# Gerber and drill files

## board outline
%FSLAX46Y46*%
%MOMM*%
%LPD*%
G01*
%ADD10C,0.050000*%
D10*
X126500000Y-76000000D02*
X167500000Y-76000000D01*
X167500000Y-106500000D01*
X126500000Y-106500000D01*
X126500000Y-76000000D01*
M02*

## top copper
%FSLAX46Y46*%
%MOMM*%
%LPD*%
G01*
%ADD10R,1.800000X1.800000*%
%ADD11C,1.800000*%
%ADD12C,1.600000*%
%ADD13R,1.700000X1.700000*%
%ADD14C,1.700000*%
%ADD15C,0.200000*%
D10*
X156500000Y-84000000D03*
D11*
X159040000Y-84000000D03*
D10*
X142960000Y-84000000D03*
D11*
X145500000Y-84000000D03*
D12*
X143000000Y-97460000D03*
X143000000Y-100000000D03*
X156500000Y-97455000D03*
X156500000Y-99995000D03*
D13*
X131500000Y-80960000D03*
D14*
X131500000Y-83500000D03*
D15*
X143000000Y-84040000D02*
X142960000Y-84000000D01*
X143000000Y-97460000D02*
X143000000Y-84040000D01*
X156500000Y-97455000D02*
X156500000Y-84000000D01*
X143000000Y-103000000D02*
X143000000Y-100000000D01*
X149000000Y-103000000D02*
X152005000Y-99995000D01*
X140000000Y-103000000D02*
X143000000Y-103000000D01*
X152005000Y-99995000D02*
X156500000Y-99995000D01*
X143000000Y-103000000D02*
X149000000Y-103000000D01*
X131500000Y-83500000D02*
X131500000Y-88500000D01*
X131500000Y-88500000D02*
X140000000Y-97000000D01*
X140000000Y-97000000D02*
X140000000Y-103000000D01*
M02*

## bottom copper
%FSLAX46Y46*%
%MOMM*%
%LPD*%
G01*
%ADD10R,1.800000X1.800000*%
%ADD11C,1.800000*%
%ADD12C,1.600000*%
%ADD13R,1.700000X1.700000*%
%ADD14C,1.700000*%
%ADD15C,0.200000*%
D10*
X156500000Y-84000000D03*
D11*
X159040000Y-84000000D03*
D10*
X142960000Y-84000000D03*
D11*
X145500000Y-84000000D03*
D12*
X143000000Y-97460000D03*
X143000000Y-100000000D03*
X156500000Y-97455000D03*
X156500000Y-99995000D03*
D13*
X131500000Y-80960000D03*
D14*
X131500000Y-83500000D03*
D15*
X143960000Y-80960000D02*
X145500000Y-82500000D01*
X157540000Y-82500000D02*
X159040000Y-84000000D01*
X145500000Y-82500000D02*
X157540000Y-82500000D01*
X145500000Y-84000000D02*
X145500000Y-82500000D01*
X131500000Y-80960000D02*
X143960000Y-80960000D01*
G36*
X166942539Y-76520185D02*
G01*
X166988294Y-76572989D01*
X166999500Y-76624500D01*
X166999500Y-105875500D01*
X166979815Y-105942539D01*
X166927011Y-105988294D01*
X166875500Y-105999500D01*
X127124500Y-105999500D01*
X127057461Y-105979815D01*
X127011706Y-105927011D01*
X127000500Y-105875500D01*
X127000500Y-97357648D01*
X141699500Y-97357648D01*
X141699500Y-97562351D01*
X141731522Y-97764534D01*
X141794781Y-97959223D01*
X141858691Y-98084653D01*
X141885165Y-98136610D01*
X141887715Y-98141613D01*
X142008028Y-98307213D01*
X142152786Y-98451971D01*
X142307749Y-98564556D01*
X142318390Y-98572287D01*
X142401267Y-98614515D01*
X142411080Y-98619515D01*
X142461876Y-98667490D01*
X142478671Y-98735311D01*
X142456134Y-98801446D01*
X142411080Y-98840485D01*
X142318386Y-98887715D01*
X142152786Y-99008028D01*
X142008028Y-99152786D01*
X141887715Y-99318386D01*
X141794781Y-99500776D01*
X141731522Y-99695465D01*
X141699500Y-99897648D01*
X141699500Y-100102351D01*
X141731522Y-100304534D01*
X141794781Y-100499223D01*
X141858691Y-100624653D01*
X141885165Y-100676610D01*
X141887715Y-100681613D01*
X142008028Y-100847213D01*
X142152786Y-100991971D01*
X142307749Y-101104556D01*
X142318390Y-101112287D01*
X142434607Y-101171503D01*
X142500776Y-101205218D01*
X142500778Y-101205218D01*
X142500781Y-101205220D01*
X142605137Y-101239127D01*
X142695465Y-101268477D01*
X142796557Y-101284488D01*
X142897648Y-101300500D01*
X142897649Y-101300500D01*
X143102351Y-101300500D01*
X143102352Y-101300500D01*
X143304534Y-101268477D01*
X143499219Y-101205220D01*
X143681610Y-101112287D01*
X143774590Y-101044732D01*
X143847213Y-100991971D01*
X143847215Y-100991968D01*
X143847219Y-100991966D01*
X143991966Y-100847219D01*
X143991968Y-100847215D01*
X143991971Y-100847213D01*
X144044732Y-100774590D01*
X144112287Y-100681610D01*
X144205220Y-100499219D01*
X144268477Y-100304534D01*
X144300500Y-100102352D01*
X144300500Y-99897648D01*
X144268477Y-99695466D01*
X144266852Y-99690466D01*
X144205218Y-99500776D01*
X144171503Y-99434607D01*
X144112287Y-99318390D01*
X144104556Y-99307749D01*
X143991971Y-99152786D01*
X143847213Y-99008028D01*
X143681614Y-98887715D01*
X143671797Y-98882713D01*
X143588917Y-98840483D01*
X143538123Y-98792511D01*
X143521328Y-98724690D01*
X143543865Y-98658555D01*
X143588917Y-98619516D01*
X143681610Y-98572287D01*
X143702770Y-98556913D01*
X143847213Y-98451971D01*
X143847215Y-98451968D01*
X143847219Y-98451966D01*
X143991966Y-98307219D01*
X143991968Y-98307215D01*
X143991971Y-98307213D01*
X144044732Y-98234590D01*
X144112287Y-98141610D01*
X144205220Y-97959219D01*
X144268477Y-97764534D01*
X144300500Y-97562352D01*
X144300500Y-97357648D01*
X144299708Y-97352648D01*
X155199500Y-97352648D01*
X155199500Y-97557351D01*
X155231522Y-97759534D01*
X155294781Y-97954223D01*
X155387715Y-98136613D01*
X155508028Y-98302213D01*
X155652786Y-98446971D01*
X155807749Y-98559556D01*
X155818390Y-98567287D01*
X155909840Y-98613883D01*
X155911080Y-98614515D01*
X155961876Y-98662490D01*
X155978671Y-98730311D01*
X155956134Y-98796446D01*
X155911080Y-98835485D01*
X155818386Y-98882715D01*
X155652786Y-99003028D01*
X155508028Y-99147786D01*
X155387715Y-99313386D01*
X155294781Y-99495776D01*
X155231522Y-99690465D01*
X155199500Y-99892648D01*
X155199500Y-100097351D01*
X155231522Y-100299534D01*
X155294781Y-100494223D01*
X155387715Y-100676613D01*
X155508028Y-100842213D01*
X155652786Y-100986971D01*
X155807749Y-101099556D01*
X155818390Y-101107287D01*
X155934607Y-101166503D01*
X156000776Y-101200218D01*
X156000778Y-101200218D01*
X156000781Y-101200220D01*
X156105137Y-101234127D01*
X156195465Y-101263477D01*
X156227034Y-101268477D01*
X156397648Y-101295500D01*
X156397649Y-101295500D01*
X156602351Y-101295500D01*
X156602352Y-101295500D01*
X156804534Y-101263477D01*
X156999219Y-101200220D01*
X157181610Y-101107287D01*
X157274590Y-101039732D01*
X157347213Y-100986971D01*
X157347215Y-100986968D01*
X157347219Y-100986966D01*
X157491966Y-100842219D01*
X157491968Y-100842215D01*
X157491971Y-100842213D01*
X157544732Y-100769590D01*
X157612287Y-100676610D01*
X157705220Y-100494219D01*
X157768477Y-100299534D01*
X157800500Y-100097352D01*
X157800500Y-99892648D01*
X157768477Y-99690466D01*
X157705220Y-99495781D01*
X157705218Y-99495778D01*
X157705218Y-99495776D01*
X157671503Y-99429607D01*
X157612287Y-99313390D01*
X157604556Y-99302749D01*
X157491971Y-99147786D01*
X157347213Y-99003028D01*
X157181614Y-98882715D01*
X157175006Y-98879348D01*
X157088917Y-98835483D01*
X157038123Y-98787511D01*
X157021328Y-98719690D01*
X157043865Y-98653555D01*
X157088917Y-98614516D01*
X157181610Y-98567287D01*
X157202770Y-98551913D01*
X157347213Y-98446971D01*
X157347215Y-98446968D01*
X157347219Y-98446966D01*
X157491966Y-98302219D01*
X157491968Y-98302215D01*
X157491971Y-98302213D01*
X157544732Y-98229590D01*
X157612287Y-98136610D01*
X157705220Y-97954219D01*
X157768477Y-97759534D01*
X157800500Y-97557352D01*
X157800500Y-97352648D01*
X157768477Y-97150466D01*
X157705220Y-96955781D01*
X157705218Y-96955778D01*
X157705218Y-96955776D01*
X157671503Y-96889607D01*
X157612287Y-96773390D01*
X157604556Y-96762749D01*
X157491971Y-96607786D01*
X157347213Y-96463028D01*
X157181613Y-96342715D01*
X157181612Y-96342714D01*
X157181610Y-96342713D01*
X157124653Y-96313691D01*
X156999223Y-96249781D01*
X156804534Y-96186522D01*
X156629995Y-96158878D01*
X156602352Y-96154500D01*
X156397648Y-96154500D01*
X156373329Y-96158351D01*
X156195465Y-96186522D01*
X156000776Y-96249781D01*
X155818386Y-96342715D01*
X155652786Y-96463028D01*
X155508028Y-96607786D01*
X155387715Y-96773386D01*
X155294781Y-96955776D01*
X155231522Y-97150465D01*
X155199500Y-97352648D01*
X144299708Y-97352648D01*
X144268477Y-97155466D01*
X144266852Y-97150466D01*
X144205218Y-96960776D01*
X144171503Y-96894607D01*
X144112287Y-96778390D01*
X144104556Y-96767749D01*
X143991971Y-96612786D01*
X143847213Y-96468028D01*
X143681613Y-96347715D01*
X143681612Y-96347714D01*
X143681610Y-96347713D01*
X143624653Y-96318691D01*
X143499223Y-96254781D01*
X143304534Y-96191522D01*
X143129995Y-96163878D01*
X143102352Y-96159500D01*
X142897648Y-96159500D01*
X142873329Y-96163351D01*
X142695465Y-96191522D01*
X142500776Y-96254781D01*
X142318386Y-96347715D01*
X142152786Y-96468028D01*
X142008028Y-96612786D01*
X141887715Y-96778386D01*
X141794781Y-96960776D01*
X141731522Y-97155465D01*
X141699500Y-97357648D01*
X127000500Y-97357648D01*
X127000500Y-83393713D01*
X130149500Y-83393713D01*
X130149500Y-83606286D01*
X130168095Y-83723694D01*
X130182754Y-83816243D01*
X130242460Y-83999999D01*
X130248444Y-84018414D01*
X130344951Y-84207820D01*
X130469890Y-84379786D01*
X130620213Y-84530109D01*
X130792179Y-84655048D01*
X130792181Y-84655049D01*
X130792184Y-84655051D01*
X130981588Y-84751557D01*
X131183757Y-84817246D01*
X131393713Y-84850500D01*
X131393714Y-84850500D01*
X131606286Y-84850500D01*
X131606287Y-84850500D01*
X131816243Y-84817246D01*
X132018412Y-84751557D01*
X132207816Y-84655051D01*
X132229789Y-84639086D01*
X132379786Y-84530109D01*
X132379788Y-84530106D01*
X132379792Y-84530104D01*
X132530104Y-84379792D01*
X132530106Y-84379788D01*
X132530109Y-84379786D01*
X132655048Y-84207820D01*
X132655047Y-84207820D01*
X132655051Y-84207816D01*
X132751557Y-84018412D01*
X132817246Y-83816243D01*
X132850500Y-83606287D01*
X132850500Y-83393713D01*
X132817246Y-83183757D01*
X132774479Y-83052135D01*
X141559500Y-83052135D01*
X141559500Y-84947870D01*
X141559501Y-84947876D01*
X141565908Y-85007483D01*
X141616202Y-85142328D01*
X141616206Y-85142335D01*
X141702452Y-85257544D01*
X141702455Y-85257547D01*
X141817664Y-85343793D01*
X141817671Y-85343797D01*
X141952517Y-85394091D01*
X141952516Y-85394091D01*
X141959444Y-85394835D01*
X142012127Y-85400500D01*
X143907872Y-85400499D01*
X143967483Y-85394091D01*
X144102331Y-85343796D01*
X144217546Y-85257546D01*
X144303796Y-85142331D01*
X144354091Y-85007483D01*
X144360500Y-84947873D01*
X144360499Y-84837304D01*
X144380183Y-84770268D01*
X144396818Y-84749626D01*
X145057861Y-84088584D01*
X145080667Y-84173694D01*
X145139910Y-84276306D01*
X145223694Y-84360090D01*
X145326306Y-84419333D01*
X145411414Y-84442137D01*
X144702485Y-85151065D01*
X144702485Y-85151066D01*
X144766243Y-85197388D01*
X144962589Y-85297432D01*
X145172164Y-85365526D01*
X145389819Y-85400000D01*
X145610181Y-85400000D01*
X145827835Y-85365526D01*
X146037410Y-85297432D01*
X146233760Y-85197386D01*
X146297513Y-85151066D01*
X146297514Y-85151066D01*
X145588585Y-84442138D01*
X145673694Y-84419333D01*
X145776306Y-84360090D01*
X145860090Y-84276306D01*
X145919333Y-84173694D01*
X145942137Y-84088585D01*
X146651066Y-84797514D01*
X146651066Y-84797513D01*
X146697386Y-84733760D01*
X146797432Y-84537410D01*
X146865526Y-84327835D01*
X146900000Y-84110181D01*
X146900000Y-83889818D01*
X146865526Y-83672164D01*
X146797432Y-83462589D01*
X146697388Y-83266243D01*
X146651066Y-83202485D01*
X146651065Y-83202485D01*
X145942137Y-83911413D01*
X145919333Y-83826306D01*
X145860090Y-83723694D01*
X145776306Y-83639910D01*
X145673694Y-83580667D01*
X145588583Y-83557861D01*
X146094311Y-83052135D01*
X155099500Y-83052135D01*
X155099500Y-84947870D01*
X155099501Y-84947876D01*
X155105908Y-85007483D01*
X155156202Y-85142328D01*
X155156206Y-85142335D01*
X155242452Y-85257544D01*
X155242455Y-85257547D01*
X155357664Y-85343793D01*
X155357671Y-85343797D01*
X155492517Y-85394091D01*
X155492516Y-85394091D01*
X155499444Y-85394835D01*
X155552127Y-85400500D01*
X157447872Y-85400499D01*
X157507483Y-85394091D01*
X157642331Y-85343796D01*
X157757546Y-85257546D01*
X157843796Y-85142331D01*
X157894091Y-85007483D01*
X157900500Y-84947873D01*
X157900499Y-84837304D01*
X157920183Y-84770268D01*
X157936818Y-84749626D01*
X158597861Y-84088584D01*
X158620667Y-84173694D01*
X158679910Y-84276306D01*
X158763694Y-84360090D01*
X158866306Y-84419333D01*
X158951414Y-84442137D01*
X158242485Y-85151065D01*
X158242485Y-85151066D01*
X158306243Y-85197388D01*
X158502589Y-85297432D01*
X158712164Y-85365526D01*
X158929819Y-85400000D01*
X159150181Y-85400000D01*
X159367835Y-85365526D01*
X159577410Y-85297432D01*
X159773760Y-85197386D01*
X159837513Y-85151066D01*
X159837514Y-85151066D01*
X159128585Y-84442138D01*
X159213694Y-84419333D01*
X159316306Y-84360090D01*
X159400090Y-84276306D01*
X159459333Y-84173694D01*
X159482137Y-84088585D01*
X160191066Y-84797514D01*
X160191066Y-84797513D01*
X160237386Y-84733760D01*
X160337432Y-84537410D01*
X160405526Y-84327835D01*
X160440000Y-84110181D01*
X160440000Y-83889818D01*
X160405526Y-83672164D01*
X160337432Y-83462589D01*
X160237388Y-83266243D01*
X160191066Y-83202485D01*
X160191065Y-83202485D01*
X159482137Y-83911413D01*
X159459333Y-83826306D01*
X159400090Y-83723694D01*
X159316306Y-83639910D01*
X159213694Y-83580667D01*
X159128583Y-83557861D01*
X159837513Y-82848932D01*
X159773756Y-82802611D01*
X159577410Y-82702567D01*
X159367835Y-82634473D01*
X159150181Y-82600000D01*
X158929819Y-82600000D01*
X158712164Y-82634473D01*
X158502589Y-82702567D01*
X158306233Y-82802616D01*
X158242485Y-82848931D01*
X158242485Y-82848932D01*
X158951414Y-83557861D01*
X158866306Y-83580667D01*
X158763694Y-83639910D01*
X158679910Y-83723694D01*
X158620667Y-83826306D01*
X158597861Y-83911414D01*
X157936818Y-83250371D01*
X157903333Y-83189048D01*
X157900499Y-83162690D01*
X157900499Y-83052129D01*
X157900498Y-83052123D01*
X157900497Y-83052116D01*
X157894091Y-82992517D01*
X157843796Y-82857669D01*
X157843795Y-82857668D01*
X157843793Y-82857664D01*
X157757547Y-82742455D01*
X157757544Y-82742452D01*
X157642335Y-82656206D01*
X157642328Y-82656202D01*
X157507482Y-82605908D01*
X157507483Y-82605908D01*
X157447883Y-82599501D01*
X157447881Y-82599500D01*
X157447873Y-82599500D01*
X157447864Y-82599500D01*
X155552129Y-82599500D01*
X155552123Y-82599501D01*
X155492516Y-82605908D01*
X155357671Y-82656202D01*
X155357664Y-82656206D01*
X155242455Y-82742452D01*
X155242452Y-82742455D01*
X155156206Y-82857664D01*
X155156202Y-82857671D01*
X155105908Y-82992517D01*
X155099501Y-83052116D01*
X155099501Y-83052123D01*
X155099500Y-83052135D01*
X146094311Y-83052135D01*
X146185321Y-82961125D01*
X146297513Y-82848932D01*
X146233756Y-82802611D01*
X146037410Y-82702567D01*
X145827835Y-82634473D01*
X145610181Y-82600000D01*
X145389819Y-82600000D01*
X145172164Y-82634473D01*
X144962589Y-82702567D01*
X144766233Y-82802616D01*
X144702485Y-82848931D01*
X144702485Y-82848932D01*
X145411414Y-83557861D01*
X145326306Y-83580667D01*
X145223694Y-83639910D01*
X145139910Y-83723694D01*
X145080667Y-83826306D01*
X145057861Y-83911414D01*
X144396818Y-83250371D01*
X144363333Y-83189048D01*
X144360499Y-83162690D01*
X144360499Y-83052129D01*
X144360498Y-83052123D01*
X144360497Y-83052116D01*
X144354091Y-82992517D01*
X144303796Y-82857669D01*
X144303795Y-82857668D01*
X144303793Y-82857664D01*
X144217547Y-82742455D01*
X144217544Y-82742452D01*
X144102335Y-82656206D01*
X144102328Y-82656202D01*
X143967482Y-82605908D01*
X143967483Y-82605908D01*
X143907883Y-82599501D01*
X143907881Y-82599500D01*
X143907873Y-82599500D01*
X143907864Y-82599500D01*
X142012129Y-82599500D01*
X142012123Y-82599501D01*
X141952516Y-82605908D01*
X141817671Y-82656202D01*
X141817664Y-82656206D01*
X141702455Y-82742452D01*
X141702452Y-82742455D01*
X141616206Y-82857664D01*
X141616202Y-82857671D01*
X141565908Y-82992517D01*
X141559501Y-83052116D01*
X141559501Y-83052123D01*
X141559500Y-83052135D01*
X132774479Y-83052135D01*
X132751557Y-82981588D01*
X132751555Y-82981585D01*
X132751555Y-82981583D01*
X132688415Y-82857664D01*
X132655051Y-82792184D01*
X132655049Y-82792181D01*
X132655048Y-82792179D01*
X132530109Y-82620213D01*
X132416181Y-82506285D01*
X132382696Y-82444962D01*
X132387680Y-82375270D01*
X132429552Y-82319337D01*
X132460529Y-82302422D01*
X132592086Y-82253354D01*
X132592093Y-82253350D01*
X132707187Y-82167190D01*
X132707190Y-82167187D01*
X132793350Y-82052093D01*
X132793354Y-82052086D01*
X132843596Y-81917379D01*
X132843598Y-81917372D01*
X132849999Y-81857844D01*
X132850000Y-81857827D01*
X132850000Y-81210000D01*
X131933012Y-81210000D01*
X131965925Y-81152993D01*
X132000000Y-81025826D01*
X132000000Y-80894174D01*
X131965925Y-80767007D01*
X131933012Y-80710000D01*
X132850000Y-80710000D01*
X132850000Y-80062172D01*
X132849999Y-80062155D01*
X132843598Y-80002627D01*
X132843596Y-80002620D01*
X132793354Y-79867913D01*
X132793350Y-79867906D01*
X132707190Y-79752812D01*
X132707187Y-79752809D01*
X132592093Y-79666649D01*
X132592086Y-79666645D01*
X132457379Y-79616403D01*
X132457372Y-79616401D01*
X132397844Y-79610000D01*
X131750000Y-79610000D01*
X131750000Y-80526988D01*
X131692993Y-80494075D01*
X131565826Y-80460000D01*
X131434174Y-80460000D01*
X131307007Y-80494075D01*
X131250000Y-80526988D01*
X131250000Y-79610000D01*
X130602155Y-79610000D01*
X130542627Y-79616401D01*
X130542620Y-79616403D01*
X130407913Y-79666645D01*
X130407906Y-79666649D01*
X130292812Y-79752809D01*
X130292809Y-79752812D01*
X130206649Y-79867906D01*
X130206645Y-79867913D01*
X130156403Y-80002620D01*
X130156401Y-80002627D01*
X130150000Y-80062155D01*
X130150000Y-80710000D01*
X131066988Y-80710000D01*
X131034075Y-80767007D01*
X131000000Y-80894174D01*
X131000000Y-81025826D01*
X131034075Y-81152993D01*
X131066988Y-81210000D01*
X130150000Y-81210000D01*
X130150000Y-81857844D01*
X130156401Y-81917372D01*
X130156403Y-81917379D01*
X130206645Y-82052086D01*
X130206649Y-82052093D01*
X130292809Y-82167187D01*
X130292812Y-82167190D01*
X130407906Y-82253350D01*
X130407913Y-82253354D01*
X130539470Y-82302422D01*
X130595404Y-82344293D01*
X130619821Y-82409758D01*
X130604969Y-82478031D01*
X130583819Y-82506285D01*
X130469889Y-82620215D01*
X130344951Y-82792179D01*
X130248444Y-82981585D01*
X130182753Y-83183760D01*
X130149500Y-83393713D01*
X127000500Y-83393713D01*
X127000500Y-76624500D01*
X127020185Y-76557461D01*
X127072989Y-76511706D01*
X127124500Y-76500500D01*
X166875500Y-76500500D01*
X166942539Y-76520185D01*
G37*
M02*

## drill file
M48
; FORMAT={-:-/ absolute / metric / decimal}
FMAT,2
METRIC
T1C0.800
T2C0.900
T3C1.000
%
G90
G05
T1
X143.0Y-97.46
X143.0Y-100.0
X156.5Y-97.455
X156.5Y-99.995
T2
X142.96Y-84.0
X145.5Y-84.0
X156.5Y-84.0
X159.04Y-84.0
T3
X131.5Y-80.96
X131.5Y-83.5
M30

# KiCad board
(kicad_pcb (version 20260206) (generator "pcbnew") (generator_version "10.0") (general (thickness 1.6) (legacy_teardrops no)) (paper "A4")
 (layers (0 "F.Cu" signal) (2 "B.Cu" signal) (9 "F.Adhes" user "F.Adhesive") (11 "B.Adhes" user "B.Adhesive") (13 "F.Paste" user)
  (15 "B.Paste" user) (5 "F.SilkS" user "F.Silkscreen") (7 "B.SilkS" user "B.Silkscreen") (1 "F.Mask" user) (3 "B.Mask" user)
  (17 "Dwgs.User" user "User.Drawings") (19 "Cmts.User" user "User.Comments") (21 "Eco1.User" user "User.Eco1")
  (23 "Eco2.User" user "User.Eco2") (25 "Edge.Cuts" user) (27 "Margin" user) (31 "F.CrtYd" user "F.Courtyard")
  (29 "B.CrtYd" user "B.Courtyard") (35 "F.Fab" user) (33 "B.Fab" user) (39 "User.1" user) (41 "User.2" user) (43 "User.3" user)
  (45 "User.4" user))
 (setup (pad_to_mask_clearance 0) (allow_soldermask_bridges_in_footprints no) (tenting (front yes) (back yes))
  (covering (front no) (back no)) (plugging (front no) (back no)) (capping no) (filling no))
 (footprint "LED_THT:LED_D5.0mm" (layer "F.Cu") (at 156.5 84)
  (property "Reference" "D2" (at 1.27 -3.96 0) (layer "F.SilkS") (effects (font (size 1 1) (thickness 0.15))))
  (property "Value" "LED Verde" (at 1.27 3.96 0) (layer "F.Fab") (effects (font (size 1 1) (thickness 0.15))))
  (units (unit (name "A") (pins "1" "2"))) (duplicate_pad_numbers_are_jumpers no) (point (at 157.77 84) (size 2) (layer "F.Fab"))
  (pad "1" thru_hole rect (at 0 0) (size 1.8 1.8) (drill 0.9) (layers "*.Cu" "*.Mask") (remove_unused_layers no) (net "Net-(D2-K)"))
  (pad "2" thru_hole circle (at 2.54 0) (size 1.8 1.8) (drill 0.9) (layers "*.Cu" "*.Mask") (remove_unused_layers no) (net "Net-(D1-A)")))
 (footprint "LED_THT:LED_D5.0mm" (layer "F.Cu") (at 142.96 84)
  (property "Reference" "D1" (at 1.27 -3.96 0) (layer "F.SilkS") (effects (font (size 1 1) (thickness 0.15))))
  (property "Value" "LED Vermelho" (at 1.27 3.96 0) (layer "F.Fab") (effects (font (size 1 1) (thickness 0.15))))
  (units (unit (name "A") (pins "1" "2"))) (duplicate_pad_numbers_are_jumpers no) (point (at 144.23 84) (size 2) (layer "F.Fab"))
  (pad "1" thru_hole rect (at 0 0) (size 1.8 1.8) (drill 0.9) (layers "*.Cu" "*.Mask") (remove_unused_layers no) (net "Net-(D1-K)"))
  (pad "2" thru_hole circle (at 2.54 0) (size 1.8 1.8) (drill 0.9) (layers "*.Cu" "*.Mask") (remove_unused_layers no) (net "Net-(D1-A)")))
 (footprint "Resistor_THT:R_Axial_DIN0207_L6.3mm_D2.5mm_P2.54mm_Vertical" (layer "F.Cu") (at 143 97.46 -90)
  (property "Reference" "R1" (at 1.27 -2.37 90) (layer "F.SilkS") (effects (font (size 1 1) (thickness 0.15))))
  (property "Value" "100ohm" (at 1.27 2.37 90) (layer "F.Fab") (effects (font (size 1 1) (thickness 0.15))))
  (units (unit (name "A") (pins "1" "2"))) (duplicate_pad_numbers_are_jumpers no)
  (pad "1" thru_hole circle (at 0 0 270) (size 1.6 1.6) (drill 0.8) (layers "*.Cu" "*.Mask") (remove_unused_layers no) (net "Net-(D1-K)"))
  (pad "2" thru_hole circle (at 2.54 0 270) (size 1.6 1.6) (drill 0.8) (layers "*.Cu" "*.Mask") (remove_unused_layers no)
   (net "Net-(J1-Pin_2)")))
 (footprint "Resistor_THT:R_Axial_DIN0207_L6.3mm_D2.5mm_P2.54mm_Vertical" (layer "F.Cu") (at 156.5 97.455 -90)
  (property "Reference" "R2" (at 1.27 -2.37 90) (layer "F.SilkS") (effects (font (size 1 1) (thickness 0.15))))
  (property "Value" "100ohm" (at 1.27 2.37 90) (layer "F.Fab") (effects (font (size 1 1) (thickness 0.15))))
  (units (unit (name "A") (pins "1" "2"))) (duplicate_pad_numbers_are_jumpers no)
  (pad "1" thru_hole circle (at 0 0 270) (size 1.6 1.6) (drill 0.8) (layers "*.Cu" "*.Mask") (remove_unused_layers no) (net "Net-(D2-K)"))
  (pad "2" thru_hole circle (at 2.54 0 270) (size 1.6 1.6) (drill 0.8) (layers "*.Cu" "*.Mask") (remove_unused_layers no)
   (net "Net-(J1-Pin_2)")))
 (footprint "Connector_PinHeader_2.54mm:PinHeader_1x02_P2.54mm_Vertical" (layer "F.Cu") (at 131.5 80.96)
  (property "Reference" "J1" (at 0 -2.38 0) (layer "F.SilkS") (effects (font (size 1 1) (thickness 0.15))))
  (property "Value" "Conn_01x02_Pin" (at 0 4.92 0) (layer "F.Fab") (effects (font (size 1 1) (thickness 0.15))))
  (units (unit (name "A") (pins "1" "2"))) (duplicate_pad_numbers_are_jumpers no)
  (pad "1" thru_hole rect (at 0 0) (size 1.7 1.7) (drill 1) (layers "*.Cu" "*.Mask") (remove_unused_layers no) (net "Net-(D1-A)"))
  (pad "2" thru_hole circle (at 0 2.54) (size 1.7 1.7) (drill 1) (layers "*.Cu" "*.Mask") (remove_unused_layers no) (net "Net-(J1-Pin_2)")))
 (gr_rect (start 126.5 76) (end 167.5 106.5) (stroke (width 0.05) (type default)) (fill no) (layer "Edge.Cuts"))
 (segment (start 156.5 97.455) (end 156.5 84) (width 0.2) (layer "F.Cu") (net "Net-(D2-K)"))
 (segment (start 143.96 80.96) (end 145.5 82.5) (width 0.2) (layer "B.Cu") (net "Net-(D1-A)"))
 (segment (start 157.54 82.5) (end 159.04 84) (width 0.2) (layer "B.Cu") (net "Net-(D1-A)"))
 (segment (start 145.5 82.5) (end 157.54 82.5) (width 0.2) (layer "B.Cu") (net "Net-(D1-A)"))
 (segment (start 145.5 84) (end 145.5 82.5) (width 0.2) (layer "B.Cu") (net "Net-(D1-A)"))
 (segment (start 131.5 80.96) (end 143.96 80.96) (width 0.2) (layer "B.Cu") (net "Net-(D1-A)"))
 (segment (start 143 84.04) (end 142.96 84) (width 0.2) (layer "F.Cu") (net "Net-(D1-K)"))
 (segment (start 143 97.46) (end 143 84.04) (width 0.2) (layer "F.Cu") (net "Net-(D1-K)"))
 (segment (start 143 103) (end 143 100) (width 0.2) (layer "F.Cu") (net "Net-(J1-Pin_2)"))
 (segment (start 149 103) (end 152.005 99.995) (width 0.2) (layer "F.Cu") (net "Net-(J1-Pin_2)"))
 (segment (start 140 103) (end 143 103) (width 0.2) (layer "F.Cu") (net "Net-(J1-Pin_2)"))
 (segment (start 152.005 99.995) (end 156.5 99.995) (width 0.2) (layer "F.Cu") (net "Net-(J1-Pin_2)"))
 (segment (start 143 103) (end 149 103) (width 0.2) (layer "F.Cu") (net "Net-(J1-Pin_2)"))
 (segment (start 131.5 83.5) (end 131.5 88.5) (width 0.2) (layer "F.Cu") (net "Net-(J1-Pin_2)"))
 (segment (start 131.5 88.5) (end 140 97) (width 0.2) (layer "F.Cu") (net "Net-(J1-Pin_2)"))
 (segment (start 140 97) (end 140 103) (width 0.2) (layer "F.Cu") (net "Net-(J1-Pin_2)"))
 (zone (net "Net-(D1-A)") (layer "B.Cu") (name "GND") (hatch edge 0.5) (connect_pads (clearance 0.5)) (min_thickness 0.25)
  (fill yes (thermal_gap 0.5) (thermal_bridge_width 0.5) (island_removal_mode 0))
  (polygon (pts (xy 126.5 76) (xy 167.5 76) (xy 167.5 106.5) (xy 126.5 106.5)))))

